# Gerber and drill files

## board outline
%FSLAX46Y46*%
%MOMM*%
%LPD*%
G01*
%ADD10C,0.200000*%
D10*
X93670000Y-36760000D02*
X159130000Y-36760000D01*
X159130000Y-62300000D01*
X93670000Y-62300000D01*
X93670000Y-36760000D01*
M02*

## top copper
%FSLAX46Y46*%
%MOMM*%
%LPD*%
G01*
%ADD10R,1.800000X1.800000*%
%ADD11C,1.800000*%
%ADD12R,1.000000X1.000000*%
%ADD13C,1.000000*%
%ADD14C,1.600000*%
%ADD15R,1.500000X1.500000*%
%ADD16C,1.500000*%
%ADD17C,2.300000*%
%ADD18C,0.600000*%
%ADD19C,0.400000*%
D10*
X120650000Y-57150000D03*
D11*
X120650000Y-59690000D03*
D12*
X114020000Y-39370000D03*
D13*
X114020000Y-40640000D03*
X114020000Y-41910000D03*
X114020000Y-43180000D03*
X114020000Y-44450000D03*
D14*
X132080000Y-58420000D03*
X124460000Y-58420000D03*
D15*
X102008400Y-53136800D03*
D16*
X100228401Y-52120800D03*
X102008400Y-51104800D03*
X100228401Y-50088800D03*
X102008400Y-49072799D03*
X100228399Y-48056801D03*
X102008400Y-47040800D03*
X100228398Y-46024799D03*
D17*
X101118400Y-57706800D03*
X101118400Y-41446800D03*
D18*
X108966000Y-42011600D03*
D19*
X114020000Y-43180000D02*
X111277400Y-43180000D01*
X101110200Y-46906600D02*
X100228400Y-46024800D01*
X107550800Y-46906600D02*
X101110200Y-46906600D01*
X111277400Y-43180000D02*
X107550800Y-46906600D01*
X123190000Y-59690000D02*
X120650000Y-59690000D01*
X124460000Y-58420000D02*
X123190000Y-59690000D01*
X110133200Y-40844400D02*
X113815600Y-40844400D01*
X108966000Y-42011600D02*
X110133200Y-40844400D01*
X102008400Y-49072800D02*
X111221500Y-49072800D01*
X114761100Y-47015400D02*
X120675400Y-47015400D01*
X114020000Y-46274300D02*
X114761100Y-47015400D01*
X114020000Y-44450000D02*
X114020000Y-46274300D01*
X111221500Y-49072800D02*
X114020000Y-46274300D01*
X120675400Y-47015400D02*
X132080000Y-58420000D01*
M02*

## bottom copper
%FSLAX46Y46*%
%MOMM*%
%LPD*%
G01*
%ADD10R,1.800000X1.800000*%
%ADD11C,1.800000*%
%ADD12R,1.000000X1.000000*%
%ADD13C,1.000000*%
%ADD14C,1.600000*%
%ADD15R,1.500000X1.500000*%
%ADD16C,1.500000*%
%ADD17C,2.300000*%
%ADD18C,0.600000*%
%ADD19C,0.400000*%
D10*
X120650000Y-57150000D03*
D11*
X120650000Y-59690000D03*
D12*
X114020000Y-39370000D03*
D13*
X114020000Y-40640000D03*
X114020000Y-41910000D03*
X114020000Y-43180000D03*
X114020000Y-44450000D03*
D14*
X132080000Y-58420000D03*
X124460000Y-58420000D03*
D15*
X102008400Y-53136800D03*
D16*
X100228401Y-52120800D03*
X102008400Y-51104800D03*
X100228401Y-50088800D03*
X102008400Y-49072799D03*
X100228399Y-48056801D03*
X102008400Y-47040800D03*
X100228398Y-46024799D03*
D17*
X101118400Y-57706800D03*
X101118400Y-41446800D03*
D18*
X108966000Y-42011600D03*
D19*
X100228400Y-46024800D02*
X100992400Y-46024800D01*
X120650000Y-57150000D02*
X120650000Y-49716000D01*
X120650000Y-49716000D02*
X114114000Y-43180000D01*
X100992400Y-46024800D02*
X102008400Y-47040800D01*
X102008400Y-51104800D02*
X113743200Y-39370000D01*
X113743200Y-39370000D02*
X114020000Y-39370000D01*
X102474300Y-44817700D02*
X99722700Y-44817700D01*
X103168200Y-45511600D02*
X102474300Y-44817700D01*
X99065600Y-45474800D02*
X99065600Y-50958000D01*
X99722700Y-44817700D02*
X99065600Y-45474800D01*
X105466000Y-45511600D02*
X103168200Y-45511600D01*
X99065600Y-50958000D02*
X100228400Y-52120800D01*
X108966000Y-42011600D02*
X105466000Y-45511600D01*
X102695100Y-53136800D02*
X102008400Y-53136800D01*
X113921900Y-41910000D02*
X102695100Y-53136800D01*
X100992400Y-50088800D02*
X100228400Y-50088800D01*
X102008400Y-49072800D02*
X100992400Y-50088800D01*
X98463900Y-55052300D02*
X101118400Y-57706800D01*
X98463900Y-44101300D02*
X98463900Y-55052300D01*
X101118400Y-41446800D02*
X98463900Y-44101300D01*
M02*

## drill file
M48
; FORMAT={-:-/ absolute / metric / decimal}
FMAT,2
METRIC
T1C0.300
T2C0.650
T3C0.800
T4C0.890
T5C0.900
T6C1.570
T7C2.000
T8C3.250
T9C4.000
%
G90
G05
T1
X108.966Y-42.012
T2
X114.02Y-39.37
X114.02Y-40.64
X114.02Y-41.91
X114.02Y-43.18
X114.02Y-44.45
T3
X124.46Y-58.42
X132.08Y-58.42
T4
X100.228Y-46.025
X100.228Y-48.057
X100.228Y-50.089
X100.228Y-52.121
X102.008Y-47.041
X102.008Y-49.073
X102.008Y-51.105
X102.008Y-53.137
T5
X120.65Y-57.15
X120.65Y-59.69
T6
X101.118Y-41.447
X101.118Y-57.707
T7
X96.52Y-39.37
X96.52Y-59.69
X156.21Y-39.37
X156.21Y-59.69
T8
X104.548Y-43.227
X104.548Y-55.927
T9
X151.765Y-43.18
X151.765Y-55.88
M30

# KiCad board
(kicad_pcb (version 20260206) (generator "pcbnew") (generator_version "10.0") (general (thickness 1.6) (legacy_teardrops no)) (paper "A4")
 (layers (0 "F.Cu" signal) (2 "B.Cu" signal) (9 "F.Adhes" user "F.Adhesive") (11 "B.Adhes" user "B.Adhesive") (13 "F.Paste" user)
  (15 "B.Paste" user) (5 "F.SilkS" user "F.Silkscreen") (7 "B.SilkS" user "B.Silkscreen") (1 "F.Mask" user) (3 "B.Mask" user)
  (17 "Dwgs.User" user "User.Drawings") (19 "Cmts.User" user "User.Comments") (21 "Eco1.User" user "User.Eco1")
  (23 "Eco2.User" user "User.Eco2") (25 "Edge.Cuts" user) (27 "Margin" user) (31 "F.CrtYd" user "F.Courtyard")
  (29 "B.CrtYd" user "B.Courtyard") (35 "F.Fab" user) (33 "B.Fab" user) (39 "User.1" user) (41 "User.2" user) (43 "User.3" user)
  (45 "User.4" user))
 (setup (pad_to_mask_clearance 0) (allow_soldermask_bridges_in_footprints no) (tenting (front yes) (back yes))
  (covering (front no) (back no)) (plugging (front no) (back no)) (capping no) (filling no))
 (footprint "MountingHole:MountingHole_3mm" (layer "F.Cu") (at 151.765 43.18)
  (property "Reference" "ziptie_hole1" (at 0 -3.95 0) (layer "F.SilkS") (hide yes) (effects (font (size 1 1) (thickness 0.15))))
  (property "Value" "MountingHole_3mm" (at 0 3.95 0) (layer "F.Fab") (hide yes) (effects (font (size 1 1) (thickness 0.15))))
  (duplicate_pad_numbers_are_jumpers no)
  (pad "" np_thru_hole circle (at 0 0) (size 4 4) (drill 4) (layers "*.Cu" "*.Mask")))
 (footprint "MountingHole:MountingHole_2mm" (layer "F.Cu") (at 156.21 59.69 90)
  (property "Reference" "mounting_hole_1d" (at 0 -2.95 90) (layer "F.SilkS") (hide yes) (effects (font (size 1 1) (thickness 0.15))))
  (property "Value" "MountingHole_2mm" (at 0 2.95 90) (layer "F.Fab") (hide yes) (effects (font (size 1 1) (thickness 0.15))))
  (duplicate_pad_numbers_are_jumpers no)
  (pad "" np_thru_hole circle (at 0 0 90) (size 2 2) (drill 2) (layers "*.Cu" "*.Mask")))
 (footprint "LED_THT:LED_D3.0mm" (layer "F.Cu") (at 120.65 57.15 -90)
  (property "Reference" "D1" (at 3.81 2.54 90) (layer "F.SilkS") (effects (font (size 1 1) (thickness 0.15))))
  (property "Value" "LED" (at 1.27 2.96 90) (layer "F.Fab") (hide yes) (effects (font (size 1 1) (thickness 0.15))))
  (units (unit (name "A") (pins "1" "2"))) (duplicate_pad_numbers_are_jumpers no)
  (pad "1" thru_hole rect (at 0 0 270) (size 1.8 1.8) (drill 0.9) (layers "*.Cu" "*.Mask") (remove_unused_layers no) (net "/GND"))
  (pad "2" thru_hole circle (at 2.54 0 270) (size 1.8 1.8) (drill 0.9) (layers "*.Cu" "*.Mask") (remove_unused_layers no) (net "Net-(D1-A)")))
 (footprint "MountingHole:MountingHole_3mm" (layer "F.Cu") (at 151.765 55.88)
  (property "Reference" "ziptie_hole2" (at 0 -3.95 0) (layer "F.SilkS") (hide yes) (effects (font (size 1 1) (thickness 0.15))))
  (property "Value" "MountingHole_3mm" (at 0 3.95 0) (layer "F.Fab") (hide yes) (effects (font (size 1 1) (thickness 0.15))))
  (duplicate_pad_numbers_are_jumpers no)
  (pad "" np_thru_hole circle (at 0 0) (size 4 4) (drill 4) (layers "*.Cu" "*.Mask")))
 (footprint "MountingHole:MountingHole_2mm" (layer "F.Cu") (at 156.21 39.37 90)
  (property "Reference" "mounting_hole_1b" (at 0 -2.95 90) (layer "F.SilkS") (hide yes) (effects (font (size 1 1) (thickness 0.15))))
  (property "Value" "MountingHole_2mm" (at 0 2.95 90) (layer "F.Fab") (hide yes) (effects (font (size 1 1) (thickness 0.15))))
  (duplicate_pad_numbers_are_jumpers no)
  (pad "" np_thru_hole circle (at 0 0 90) (size 2 2) (drill 2) (layers "*.Cu" "*.Mask")))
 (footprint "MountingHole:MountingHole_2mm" (layer "F.Cu") (at 96.52 39.37 90)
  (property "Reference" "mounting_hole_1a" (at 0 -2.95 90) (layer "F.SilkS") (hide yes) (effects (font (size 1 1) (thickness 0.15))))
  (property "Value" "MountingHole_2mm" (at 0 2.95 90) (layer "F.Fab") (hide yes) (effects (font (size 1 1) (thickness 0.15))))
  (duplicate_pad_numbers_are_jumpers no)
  (pad "" np_thru_hole circle (at 0 0 90) (size 2 2) (drill 2) (layers "*.Cu" "*.Mask")))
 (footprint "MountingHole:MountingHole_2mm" (layer "F.Cu") (at 96.52 59.69 90)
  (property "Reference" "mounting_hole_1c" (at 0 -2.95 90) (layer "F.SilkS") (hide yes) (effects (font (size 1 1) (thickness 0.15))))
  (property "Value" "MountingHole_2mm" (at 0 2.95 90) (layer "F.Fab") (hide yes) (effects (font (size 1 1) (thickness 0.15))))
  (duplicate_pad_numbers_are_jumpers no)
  (pad "" np_thru_hole circle (at 0 0 90) (size 2 2) (drill 2) (layers "*.Cu" "*.Mask")))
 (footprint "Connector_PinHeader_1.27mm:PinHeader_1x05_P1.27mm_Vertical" (layer "F.Cu") (at 114.02 39.37)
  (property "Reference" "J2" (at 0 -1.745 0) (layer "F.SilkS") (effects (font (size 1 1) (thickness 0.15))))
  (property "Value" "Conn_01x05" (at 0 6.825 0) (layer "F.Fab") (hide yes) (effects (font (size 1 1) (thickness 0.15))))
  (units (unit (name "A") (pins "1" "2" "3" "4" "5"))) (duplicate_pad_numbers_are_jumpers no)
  (pad "1" thru_hole rect (at 0 0) (size 1 1) (drill 0.65) (layers "*.Cu" "*.Mask") (remove_unused_layers no) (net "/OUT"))
  (pad "2" thru_hole circle (at 0 1.27) (size 1 1) (drill 0.65) (layers "*.Cu" "*.Mask") (remove_unused_layers no) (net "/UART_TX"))
  (pad "3" thru_hole circle (at 0 2.54) (size 1 1) (drill 0.65) (layers "*.Cu" "*.Mask") (remove_unused_layers no) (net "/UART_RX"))
  (pad "4" thru_hole circle (at 0 3.81) (size 1 1) (drill 0.65) (layers "*.Cu" "*.Mask") (remove_unused_layers no) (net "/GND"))
  (pad "5" thru_hole circle (at 0 5.08) (size 1 1) (drill 0.65) (layers "*.Cu" "*.Mask") (remove_unused_layers no) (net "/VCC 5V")))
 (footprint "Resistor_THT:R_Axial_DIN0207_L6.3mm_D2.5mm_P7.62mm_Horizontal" (layer "B.Cu") (at 132.08 58.42 180)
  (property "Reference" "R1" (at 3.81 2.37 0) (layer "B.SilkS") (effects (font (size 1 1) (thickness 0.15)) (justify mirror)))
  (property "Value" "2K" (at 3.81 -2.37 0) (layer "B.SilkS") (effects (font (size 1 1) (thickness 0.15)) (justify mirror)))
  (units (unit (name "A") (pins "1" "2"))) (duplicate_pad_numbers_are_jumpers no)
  (pad "1" thru_hole circle (at 0 0 180) (size 1.6 1.6) (drill 0.8) (layers "*.Cu" "*.Mask") (remove_unused_layers no) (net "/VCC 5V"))
  (pad "2" thru_hole circle (at 7.62 0 180) (size 1.6 1.6) (drill 0.8) (layers "*.Cu" "*.Mask") (remove_unused_layers no) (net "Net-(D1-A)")))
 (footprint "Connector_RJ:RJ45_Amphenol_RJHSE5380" (layer "B.Cu") (at 102.0084 53.1368 90)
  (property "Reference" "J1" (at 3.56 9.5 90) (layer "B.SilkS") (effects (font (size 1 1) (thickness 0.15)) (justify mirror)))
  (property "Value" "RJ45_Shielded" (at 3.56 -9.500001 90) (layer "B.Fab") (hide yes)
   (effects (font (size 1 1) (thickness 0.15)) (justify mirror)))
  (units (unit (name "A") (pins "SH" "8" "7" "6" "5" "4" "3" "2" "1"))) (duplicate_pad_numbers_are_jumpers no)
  (pad "" np_thru_hole circle (at -2.79 2.54 90) (size 3.25 3.25) (drill 3.25) (layers "*.Cu" "*.Mask"))
  (pad "" np_thru_hole circle (at 9.91 2.54 90) (size 3.25 3.25) (drill 3.25) (layers "*.Cu" "*.Mask"))
  (pad "1" thru_hole rect (at 0 0 90) (size 1.5 1.5) (drill 0.89) (layers "*.Cu" "*.Mask") (remove_unused_layers no) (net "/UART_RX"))
  (pad "2" thru_hole circle (at 1.016 -1.779999 90) (size 1.5 1.5) (drill 0.89) (layers "*.Cu" "*.Mask") (remove_unused_layers no)
   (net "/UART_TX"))
  (pad "3" thru_hole circle (at 2.032 0 90) (size 1.5 1.5) (drill 0.89) (layers "*.Cu" "*.Mask") (remove_unused_layers no) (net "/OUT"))
  (pad "4" thru_hole circle (at 3.048 -1.779999 90) (size 1.5 1.5) (drill 0.89) (layers "*.Cu" "*.Mask") (remove_unused_layers no)
   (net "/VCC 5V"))
  (pad "5" thru_hole circle (at 4.064001 0 90) (size 1.5 1.5) (drill 0.89) (layers "*.Cu" "*.Mask") (remove_unused_layers no)
   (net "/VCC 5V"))
  (pad "6" thru_hole circle (at 5.079999 -1.780001 90) (size 1.5 1.5) (drill 0.89) (layers "*.Cu" "*.Mask") (remove_unused_layers no)
   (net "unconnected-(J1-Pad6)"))
  (pad "7" thru_hole circle (at 6.096 0 90) (size 1.5 1.5) (drill 0.89) (layers "*.Cu" "*.Mask") (remove_unused_layers no) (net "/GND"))
  (pad "8" thru_hole circle (at 7.112001 -1.780002 90) (size 1.5 1.5) (drill 0.89) (layers "*.Cu" "*.Mask") (remove_unused_layers no)
   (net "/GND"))
  (pad "SH" thru_hole circle (at -4.57 -0.89 90) (size 2.3 2.3) (drill 1.57) (layers "*.Cu" "*.Mask") (remove_unused_layers no)
   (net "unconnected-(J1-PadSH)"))
  (pad "SH" thru_hole circle (at 11.69 -0.89 90) (size 2.3 2.3) (drill 1.57) (layers "*.Cu" "*.Mask") (remove_unused_layers no)
   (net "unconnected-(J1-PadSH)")))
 (gr_rect (start 93.67 36.76) (end 159.13 62.3) (stroke (width 0.2) (type solid)) (fill no) (layer "Edge.Cuts"))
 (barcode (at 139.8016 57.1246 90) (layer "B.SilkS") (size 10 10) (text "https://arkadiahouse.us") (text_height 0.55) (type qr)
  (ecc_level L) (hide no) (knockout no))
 (segment (start 114.02 43.18) (end 111.2774 43.18) (width 0.4) (layer "F.Cu") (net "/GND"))
 (segment (start 101.1102 46.9066) (end 100.2284 46.0248) (width 0.4) (layer "F.Cu") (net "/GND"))
 (segment (start 107.5508 46.9066) (end 101.1102 46.9066) (width 0.4) (layer "F.Cu") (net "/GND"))
 (segment (start 111.2774 43.18) (end 107.5508 46.9066) (width 0.4) (layer "F.Cu") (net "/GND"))
 (segment (start 100.2284 46.0248) (end 100.9924 46.0248) (width 0.4) (layer "B.Cu") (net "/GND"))
 (segment (start 120.65 57.15) (end 120.65 49.716) (width 0.4) (layer "B.Cu") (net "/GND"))
 (segment (start 120.65 49.716) (end 114.114 43.18) (width 0.4) (layer "B.Cu") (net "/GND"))
 (segment (start 100.9924 46.0248) (end 102.0084 47.0408) (width 0.4) (layer "B.Cu") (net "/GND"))
 (segment (start 123.19 59.69) (end 120.65 59.69) (width 0.4) (layer "F.Cu") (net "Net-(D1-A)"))
 (segment (start 124.46 58.42) (end 123.19 59.69) (width 0.4) (layer "F.Cu") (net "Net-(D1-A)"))
 (segment (start 102.0084 51.1048) (end 113.7432 39.37) (width 0.4) (layer "B.Cu") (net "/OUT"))
 (segment (start 113.7432 39.37) (end 114.02 39.37) (width 0.4) (layer "B.Cu") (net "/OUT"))
 (segment (start 110.1332 40.8444) (end 113.8156 40.8444) (width 0.4) (layer "F.Cu") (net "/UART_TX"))
 (segment (start 108.966 42.0116) (end 110.1332 40.8444) (width 0.4) (layer "F.Cu") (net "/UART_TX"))
 (via (at 108.966 42.0116) (size 0.6) (drill 0.3) (layers "F.Cu" "B.Cu") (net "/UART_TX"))
 (segment (start 102.4743 44.8177) (end 99.7227 44.8177) (width 0.4) (layer "B.Cu") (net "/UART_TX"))
 (segment (start 103.1682 45.5116) (end 102.4743 44.8177) (width 0.4) (layer "B.Cu") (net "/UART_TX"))
 (segment (start 99.0656 45.4748) (end 99.0656 50.958) (width 0.4) (layer "B.Cu") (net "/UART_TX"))
 (segment (start 99.7227 44.8177) (end 99.0656 45.4748) (width 0.4) (layer "B.Cu") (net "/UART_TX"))
 (segment (start 105.466 45.5116) (end 103.1682 45.5116) (width 0.4) (layer "B.Cu") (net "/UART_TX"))
 (segment (start 99.0656 50.958) (end 100.2284 52.1208) (width 0.4) (layer "B.Cu") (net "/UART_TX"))
 (segment (start 108.966 42.0116) (end 105.466 45.5116) (width 0.4) (layer "B.Cu") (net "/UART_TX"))
 (segment (start 102.6951 53.1368) (end 102.0084 53.1368) (width 0.4) (layer "B.Cu") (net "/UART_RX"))
 (segment (start 113.9219 41.91) (end 102.6951 53.1368) (width 0.4) (layer "B.Cu") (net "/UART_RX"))
 (segment (start 102.0084 49.0728) (end 111.2215 49.0728) (width 0.4) (layer "F.Cu") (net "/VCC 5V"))
 (segment (start 114.7611 47.0154) (end 120.6754 47.0154) (width 0.4) (layer "F.Cu") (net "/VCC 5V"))
 (segment (start 114.02 46.2743) (end 114.7611 47.0154) (width 0.4) (layer "F.Cu") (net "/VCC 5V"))
 (segment (start 114.02 44.45) (end 114.02 46.2743) (width 0.4) (layer "F.Cu") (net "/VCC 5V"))
 (segment (start 111.2215 49.0728) (end 114.02 46.2743) (width 0.4) (layer "F.Cu") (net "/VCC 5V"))
 (segment (start 120.6754 47.0154) (end 132.08 58.42) (width 0.4) (layer "F.Cu") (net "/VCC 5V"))
 (segment (start 100.9924 50.0888) (end 100.2284 50.0888) (width 0.4) (layer "B.Cu") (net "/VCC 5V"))
 (segment (start 102.0084 49.0728) (end 100.9924 50.0888) (width 0.4) (layer "B.Cu") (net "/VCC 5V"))
 (segment (start 98.4639 55.0523) (end 101.1184 57.7068) (width 0.4) (layer "B.Cu") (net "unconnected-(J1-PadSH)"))
 (segment (start 98.4639 44.1013) (end 98.4639 55.0523) (width 0.4) (layer "B.Cu") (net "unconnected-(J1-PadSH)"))
 (segment (start 101.1184 41.4468) (end 98.4639 44.1013) (width 0.4) (layer "B.Cu") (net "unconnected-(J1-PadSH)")))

